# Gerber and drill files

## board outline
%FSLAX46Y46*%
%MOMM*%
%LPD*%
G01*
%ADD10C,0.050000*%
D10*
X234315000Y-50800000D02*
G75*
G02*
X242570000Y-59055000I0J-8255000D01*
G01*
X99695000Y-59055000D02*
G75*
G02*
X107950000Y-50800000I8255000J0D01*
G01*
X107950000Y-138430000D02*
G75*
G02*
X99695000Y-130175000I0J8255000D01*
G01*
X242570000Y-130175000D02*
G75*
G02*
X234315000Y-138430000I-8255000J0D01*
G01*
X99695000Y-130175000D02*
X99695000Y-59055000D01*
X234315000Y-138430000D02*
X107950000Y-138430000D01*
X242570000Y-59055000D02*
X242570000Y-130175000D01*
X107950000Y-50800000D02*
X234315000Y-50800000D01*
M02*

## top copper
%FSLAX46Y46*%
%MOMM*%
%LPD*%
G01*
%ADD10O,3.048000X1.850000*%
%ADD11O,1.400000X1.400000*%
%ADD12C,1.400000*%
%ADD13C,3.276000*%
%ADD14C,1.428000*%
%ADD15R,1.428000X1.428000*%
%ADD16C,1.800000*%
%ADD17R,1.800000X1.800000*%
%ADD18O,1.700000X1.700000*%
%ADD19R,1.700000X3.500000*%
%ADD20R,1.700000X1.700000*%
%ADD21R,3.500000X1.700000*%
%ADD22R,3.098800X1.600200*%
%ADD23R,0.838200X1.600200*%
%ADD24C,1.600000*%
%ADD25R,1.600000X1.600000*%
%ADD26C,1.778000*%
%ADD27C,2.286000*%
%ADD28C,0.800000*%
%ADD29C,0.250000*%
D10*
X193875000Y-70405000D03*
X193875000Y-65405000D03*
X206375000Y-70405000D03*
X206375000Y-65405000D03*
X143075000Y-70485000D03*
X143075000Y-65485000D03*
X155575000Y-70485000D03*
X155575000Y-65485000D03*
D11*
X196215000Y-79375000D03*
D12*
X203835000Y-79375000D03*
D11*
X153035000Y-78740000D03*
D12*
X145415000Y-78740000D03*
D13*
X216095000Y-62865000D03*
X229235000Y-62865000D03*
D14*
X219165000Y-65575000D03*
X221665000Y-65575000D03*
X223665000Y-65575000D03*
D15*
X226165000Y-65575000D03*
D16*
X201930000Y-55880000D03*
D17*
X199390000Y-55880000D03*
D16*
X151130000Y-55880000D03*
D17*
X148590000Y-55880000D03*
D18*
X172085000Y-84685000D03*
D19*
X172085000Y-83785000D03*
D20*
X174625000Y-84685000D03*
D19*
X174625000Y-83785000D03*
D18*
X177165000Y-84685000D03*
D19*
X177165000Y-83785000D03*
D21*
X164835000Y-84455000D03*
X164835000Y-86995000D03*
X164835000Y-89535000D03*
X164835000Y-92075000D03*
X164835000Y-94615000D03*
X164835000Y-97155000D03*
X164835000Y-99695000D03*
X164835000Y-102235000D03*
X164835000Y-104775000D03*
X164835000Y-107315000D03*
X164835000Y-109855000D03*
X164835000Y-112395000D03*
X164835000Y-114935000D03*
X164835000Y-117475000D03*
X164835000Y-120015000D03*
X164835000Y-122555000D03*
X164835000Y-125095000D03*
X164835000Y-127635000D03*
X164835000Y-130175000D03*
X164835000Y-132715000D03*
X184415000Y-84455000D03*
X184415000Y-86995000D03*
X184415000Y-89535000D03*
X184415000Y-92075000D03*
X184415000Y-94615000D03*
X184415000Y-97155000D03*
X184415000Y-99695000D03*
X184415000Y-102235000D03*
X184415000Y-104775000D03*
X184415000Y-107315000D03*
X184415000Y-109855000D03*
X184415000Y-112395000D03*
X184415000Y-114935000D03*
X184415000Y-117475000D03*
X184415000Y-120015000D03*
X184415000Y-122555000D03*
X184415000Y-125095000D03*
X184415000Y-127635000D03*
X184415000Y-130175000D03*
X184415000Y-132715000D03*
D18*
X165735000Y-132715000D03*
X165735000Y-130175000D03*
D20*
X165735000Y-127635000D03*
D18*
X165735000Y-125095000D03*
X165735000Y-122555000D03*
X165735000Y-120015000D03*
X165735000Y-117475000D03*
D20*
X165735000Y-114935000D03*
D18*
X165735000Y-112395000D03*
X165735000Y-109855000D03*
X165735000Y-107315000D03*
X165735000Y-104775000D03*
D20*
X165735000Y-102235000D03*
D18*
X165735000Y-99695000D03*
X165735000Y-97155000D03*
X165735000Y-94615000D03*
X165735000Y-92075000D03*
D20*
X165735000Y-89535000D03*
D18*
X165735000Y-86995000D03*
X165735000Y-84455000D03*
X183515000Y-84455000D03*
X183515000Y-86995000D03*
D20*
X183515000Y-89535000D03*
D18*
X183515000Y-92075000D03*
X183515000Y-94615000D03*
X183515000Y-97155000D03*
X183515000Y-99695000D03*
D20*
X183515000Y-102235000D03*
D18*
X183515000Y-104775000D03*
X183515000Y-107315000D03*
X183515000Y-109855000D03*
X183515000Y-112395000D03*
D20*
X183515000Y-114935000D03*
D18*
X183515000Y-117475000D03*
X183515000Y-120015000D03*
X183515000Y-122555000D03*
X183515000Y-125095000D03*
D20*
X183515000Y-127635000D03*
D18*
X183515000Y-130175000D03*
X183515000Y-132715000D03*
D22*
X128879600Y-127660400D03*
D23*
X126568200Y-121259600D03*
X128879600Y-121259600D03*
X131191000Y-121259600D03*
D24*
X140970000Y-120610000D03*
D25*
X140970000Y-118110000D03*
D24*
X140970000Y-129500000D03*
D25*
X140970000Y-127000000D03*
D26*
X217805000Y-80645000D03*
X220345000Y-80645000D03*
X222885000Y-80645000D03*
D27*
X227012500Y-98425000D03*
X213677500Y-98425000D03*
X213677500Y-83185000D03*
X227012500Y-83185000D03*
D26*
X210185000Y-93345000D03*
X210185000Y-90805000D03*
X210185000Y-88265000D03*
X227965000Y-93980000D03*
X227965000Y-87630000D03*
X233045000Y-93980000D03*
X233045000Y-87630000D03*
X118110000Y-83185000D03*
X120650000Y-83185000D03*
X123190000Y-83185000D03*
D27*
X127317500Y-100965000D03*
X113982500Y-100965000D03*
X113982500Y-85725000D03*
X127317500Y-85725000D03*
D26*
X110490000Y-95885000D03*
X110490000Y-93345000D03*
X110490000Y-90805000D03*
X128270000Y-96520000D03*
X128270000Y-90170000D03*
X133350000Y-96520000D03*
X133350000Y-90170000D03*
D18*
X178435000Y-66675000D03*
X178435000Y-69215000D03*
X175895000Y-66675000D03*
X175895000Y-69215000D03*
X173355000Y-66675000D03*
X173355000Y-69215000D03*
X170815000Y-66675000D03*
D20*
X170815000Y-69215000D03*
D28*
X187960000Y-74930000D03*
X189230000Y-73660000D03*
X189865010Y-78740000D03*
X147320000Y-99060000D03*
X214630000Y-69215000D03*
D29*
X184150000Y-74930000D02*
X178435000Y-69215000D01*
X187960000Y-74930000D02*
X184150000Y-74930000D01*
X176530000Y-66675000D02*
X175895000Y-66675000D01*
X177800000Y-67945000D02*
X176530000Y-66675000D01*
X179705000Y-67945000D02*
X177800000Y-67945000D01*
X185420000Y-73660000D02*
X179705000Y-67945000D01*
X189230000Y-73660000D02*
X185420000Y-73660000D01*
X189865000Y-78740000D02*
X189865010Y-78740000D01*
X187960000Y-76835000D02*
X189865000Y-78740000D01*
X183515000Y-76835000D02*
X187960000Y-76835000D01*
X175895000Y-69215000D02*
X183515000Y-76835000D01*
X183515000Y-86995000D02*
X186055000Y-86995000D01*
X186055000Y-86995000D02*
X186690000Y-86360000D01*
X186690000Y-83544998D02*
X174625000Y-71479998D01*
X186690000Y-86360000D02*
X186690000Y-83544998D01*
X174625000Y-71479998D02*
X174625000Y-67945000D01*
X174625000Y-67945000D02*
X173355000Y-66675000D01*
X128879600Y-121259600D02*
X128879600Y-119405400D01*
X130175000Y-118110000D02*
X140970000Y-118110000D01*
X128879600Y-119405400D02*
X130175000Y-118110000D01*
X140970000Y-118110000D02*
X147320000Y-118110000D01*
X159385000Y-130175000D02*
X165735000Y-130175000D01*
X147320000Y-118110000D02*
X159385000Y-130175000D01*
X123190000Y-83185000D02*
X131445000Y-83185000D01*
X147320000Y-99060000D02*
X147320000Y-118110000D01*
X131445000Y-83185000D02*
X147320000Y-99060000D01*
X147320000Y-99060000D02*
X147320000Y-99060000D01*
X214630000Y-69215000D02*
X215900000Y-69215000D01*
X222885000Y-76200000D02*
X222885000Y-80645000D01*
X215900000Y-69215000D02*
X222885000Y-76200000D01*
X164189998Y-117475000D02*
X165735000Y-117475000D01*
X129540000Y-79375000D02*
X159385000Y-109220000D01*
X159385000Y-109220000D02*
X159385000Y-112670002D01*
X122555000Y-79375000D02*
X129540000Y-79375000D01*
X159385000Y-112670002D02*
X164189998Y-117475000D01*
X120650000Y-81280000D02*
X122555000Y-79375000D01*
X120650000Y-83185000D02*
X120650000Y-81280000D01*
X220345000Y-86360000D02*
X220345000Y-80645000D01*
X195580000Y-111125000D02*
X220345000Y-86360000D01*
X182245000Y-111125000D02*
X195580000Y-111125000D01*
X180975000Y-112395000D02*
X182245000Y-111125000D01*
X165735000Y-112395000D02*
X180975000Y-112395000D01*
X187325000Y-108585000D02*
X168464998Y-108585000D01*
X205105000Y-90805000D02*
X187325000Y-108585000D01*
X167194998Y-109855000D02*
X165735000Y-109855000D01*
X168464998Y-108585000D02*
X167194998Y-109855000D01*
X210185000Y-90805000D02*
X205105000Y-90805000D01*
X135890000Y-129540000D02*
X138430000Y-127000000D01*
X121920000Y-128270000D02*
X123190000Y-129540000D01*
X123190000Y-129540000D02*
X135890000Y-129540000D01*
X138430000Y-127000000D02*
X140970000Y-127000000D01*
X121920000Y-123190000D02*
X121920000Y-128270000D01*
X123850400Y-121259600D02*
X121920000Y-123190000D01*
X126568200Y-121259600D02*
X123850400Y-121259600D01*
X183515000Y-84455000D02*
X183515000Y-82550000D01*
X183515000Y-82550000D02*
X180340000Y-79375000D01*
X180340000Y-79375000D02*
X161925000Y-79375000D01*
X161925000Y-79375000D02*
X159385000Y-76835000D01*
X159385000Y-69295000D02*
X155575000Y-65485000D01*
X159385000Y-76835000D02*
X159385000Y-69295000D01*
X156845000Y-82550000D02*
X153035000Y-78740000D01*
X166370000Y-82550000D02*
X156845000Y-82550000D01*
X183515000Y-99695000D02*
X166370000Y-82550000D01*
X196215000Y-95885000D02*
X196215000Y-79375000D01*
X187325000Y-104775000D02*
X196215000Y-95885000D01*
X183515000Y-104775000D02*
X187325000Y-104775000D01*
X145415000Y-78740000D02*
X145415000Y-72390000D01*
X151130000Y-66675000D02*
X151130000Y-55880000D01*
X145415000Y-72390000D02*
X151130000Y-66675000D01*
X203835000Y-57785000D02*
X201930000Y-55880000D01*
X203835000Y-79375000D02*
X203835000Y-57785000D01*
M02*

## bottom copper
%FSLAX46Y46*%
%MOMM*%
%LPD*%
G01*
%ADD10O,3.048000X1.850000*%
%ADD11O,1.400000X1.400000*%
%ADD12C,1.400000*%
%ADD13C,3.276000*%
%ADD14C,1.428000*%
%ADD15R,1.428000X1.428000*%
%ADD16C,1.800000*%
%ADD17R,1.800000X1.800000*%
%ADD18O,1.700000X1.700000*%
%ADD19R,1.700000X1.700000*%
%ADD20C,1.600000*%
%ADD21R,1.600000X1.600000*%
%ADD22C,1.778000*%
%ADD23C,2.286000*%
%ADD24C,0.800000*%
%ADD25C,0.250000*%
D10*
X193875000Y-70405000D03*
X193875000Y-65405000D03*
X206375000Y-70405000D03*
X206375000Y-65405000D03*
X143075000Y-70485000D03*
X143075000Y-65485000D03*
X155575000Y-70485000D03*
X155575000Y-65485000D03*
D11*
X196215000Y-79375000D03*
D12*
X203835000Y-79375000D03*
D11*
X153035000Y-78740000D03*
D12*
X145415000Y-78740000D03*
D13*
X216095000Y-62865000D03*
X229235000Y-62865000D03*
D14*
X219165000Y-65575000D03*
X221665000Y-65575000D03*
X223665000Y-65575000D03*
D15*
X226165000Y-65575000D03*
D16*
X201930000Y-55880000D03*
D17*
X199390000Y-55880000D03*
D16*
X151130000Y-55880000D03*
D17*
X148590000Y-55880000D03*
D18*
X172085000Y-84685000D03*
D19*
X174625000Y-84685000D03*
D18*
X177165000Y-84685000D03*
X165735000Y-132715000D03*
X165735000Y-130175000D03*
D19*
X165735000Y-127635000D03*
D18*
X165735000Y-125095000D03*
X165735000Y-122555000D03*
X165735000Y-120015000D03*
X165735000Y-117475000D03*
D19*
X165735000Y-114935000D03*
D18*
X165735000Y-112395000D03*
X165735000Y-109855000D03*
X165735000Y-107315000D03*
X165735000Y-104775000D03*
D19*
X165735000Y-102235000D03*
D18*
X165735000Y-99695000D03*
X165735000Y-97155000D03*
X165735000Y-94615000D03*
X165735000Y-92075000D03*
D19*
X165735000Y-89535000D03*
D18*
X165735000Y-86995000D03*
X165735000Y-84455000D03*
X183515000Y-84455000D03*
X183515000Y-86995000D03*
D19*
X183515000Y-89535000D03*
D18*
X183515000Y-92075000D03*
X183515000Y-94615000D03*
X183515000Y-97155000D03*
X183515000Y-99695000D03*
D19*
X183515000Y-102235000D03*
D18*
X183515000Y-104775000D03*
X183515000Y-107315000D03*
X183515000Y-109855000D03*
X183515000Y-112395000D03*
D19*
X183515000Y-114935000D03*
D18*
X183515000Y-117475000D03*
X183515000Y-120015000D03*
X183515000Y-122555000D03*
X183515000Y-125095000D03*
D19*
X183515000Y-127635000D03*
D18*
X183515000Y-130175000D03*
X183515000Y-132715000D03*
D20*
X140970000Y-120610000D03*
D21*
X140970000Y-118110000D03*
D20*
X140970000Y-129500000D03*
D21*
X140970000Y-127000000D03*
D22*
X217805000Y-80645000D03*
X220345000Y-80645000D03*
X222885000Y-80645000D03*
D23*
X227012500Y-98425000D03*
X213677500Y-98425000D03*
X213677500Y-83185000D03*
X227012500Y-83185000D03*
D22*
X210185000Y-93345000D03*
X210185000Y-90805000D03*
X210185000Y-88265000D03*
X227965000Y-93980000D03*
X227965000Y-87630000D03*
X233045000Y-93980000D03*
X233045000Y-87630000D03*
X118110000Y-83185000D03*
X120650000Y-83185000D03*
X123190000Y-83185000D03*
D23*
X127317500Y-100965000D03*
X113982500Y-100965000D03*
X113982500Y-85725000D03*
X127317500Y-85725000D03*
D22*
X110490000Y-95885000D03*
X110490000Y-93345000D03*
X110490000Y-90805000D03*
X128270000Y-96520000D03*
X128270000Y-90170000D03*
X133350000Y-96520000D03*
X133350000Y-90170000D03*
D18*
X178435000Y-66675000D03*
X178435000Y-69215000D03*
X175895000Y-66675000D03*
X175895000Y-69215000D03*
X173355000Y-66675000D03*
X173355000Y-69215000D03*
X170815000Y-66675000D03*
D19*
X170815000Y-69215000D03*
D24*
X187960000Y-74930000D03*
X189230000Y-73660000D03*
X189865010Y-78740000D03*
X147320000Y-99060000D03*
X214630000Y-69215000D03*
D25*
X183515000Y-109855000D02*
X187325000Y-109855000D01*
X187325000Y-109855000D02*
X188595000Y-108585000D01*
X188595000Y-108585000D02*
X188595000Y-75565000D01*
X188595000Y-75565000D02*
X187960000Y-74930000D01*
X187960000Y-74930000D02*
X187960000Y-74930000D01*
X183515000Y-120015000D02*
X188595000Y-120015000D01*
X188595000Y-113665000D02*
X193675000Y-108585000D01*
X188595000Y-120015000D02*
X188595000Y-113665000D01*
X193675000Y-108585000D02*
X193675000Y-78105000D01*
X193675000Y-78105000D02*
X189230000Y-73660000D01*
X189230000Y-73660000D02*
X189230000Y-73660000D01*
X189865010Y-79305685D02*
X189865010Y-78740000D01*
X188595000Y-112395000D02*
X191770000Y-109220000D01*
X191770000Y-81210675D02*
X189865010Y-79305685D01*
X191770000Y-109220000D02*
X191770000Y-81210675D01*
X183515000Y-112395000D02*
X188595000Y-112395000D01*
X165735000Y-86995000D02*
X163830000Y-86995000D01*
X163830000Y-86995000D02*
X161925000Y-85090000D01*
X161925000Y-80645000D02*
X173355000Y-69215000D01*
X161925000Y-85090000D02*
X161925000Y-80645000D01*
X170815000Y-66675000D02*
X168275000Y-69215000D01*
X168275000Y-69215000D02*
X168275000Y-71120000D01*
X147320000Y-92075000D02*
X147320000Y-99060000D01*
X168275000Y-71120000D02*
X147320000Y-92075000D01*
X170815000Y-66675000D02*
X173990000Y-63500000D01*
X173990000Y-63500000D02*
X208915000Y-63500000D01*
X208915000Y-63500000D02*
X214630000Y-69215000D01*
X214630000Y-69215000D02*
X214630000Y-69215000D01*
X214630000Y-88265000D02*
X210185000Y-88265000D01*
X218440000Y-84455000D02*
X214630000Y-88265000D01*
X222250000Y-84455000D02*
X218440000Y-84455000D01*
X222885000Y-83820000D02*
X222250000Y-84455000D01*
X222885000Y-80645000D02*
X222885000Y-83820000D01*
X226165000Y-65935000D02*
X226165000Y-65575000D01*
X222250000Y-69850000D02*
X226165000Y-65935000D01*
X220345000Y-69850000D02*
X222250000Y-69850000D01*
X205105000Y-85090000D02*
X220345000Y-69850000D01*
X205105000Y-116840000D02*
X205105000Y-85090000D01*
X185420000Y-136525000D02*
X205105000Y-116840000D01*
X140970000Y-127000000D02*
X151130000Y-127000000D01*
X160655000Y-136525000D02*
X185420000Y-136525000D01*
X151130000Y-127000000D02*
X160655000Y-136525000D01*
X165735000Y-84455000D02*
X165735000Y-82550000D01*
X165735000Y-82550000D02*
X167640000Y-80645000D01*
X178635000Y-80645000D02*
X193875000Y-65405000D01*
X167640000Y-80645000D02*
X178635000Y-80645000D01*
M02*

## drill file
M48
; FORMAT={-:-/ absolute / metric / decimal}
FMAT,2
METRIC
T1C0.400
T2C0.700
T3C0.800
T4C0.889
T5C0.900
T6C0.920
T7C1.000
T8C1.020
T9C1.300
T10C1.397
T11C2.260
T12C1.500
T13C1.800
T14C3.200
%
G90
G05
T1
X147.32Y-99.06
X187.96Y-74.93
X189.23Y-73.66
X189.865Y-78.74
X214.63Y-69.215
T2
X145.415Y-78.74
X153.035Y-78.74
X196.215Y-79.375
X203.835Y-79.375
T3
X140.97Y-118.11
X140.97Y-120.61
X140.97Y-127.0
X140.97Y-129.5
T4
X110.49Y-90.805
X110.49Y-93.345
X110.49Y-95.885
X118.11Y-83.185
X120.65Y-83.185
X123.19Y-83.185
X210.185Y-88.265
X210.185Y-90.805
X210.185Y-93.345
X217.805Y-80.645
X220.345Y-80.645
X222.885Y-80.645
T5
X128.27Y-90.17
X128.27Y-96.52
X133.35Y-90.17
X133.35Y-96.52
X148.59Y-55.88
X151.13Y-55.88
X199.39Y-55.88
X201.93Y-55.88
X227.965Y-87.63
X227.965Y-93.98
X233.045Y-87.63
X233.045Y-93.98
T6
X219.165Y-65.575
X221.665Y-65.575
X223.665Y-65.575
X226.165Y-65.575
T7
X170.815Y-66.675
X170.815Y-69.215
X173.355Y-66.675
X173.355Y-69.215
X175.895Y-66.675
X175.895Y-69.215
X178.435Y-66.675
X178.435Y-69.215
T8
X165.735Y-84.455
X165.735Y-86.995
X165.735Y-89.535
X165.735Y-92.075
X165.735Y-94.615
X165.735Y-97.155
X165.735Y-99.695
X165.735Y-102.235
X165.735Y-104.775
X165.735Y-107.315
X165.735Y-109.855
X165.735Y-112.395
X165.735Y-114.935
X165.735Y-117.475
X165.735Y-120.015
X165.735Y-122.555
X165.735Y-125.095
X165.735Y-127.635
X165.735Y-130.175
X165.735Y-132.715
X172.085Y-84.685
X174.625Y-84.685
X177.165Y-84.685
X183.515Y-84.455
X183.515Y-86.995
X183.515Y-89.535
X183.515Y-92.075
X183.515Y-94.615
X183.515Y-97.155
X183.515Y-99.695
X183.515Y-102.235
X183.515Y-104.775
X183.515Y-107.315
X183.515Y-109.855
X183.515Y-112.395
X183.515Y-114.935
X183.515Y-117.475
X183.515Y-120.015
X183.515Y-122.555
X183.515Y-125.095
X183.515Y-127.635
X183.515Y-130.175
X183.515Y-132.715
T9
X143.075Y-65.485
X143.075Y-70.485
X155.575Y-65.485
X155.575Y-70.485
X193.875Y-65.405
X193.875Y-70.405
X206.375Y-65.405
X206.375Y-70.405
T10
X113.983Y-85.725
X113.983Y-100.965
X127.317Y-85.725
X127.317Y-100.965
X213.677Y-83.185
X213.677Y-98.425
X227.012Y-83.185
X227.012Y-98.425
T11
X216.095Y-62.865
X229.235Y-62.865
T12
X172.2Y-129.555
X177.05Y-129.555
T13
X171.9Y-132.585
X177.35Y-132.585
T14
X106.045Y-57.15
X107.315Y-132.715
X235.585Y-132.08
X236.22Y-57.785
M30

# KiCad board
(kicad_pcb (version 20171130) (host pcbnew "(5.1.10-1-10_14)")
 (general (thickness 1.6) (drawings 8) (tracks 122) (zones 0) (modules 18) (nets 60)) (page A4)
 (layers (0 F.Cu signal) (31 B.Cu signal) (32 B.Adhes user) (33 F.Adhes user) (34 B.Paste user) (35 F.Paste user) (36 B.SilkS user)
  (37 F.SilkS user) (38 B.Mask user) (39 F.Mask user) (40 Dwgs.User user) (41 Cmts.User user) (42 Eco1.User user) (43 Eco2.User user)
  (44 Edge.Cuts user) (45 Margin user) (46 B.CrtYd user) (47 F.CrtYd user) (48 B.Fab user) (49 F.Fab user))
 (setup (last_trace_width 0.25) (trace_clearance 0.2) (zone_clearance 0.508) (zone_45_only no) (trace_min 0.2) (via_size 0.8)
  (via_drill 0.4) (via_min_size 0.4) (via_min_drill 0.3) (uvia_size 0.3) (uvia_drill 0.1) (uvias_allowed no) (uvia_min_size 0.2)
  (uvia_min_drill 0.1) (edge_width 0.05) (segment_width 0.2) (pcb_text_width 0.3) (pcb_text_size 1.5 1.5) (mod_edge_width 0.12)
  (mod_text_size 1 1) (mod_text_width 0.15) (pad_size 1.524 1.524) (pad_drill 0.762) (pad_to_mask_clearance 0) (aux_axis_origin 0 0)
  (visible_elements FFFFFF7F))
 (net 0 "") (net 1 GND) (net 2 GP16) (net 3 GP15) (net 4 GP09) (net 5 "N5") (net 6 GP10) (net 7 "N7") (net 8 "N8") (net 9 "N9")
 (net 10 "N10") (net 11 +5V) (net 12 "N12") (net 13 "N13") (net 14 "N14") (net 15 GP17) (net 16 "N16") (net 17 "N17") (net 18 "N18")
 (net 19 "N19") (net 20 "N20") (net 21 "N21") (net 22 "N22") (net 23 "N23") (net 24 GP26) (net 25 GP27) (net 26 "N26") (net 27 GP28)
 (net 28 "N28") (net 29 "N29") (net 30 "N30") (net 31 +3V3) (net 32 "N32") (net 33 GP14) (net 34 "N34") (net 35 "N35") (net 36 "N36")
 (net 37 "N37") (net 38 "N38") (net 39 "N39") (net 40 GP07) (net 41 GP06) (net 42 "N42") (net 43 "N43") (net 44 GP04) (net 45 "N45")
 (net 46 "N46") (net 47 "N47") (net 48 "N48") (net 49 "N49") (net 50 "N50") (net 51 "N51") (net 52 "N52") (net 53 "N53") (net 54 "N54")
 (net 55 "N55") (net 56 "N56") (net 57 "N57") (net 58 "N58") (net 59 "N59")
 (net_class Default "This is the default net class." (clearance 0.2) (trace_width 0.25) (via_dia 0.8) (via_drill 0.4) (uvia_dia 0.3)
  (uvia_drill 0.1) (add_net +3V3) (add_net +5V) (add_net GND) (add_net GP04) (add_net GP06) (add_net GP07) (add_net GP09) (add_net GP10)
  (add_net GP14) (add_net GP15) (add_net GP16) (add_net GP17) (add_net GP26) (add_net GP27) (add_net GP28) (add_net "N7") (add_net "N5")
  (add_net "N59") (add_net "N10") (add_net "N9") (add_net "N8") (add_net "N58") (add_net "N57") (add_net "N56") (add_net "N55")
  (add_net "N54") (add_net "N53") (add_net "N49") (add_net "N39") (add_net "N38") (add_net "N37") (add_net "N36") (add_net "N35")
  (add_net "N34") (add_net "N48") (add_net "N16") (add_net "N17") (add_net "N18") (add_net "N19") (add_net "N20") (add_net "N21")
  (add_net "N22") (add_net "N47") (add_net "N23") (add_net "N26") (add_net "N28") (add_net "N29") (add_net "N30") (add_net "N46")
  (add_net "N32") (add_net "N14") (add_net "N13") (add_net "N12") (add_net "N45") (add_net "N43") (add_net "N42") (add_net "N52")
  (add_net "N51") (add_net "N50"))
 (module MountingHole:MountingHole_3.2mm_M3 (layer F.Cu) (at 106.045 57.15)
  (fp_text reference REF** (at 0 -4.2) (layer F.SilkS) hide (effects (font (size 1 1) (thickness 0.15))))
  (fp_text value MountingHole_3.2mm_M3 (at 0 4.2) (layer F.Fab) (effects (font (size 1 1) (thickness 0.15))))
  (pad 1 np_thru_hole circle (at 0 0) (size 3.2 3.2) (drill 3.2) (layers *.Cu *.Mask)))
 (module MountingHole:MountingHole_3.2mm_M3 (layer F.Cu) (at 107.315 132.715)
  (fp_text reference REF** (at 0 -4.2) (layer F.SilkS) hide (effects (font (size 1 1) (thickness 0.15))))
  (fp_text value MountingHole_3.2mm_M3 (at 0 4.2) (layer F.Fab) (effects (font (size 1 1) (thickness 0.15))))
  (pad 1 np_thru_hole circle (at 0 0) (size 3.2 3.2) (drill 3.2) (layers *.Cu *.Mask)))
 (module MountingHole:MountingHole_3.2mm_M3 (layer F.Cu) (at 235.585 132.08)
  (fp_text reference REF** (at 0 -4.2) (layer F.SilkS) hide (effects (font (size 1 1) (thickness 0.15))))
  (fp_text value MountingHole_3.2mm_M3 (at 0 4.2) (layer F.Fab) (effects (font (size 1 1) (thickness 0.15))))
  (pad 1 np_thru_hole circle (at 0 0) (size 3.2 3.2) (drill 3.2) (layers *.Cu *.Mask)))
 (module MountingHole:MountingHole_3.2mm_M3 (layer F.Cu) (at 236.22 57.785)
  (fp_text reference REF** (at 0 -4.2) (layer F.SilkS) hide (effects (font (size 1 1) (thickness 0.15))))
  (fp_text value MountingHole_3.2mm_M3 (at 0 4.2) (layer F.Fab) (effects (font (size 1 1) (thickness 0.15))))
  (pad 1 np_thru_hole circle (at 0 0) (size 3.2 3.2) (drill 3.2) (layers *.Cu *.Mask)))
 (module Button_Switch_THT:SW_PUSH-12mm (layer F.Cu) (at 193.875 65.405)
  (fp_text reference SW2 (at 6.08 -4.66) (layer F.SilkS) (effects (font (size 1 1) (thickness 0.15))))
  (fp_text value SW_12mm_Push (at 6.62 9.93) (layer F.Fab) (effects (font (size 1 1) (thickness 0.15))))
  (pad 2 thru_hole oval (at 0 5) (size 3.048 1.85) (drill 1.3) (layers *.Cu *.Mask) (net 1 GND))
  (pad 1 thru_hole oval (at 0 0) (size 3.048 1.85) (drill 1.3) (layers *.Cu *.Mask) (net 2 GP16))
  (pad 2 thru_hole oval (at 12.5 5) (size 3.048 1.85) (drill 1.3) (layers *.Cu *.Mask) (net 1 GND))
  (pad 1 thru_hole oval (at 12.5 0) (size 3.048 1.85) (drill 1.3) (layers *.Cu *.Mask) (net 2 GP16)))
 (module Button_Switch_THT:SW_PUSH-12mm (layer F.Cu) (at 143.075 65.485)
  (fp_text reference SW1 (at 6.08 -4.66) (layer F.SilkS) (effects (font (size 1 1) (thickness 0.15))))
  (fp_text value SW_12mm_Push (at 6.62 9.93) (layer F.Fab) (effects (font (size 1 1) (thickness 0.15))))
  (pad 2 thru_hole oval (at 0 5) (size 3.048 1.85) (drill 1.3) (layers *.Cu *.Mask) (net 1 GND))
  (pad 1 thru_hole oval (at 0 0) (size 3.048 1.85) (drill 1.3) (layers *.Cu *.Mask) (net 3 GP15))
  (pad 2 thru_hole oval (at 12.5 5) (size 3.048 1.85) (drill 1.3) (layers *.Cu *.Mask) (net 1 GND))
  (pad 1 thru_hole oval (at 12.5 0) (size 3.048 1.85) (drill 1.3) (layers *.Cu *.Mask) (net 3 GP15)))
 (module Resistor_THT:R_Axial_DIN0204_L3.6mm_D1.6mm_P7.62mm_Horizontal (layer F.Cu) (at 203.835 79.375 180)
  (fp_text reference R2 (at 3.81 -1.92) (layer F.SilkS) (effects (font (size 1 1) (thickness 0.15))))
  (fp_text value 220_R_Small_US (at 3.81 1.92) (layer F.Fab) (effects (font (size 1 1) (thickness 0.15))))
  (pad 2 thru_hole oval (at 7.62 0 180) (size 1.4 1.4) (drill 0.7) (layers *.Cu *.Mask) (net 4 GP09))
  (pad 1 thru_hole circle (at 0 0 180) (size 1.4 1.4) (drill 0.7) (layers *.Cu *.Mask) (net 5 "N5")))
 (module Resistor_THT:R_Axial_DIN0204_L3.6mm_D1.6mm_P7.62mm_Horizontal (layer F.Cu) (at 145.415 78.74)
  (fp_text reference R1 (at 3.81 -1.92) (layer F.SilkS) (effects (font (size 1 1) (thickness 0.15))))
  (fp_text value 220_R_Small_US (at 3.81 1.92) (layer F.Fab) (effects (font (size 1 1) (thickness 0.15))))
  (pad 2 thru_hole oval (at 7.62 0) (size 1.4 1.4) (drill 0.7) (layers *.Cu *.Mask) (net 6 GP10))
  (pad 1 thru_hole circle (at 0 0) (size 1.4 1.4) (drill 0.7) (layers *.Cu *.Mask) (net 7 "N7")))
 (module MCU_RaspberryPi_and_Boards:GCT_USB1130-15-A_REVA (layer F.Cu) (at 222.665 62.865 180)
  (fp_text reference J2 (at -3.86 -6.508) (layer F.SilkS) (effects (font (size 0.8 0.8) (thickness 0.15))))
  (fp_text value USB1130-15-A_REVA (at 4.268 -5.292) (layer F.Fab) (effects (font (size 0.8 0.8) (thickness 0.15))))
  (pad S2 thru_hole circle (at 6.57 0 180) (size 3.276 3.276) (drill 2.26) (layers *.Cu *.Mask) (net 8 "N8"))
  (pad S1 thru_hole circle (at -6.57 0 180) (size 3.276 3.276) (drill 2.26) (layers *.Cu *.Mask) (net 8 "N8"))
  (pad 4 thru_hole circle (at 3.5 -2.71 180) (size 1.428 1.428) (drill 0.92) (layers *.Cu *.Mask) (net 1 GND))
  (pad 3 thru_hole circle (at 1 -2.71 180) (size 1.428 1.428) (drill 0.92) (layers *.Cu *.Mask) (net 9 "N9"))
  (pad 2 thru_hole circle (at -1 -2.71 180) (size 1.428 1.428) (drill 0.92) (layers *.Cu *.Mask) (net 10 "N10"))
  (pad 1 thru_hole rect (at -3.5 -2.71 180) (size 1.428 1.428) (drill 0.92) (layers *.Cu *.Mask) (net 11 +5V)))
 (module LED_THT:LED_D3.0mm (layer F.Cu) (at 199.39 55.88)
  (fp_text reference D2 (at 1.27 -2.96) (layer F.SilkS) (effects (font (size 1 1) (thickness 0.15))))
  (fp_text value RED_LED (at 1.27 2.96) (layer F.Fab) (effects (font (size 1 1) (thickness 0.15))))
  (pad 2 thru_hole circle (at 2.54 0) (size 1.8 1.8) (drill 0.9) (layers *.Cu *.Mask) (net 5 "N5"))
  (pad 1 thru_hole rect (at 0 0) (size 1.8 1.8) (drill 0.9) (layers *.Cu *.Mask) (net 1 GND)))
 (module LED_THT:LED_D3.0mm (layer F.Cu) (at 148.59 55.88)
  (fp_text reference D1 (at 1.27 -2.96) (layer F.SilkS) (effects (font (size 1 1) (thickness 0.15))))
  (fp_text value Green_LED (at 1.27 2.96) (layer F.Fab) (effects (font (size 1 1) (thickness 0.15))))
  (pad 2 thru_hole circle (at 2.54 0) (size 1.8 1.8) (drill 0.9) (layers *.Cu *.Mask) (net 7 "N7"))
  (pad 1 thru_hole rect (at 0 0) (size 1.8 1.8) (drill 0.9) (layers *.Cu *.Mask) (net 1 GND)))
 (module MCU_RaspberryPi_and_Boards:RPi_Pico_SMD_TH (layer F.Cu) (at 174.625 108.585 180)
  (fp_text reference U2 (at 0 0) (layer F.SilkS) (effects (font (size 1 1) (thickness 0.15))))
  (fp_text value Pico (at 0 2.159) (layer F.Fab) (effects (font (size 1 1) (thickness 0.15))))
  (pad 43 thru_hole oval (at 2.54 23.9 180) (size 1.7 1.7) (drill 1.02) (layers *.Cu *.Mask) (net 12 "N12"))
  (pad 43 smd rect (at 2.54 23.9 270) (size 3.5 1.7) (drill (offset -0.9 0)) (layers F.Cu F.Mask) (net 12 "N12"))
  (pad 42 thru_hole rect (at 0 23.9 180) (size 1.7 1.7) (drill 1.02) (layers *.Cu *.Mask) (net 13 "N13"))
  (pad 42 smd rect (at 0 23.9 270) (size 3.5 1.7) (drill (offset -0.9 0)) (layers F.Cu F.Mask) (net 13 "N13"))
  (pad 41 thru_hole oval (at -2.54 23.9 180) (size 1.7 1.7) (drill 1.02) (layers *.Cu *.Mask) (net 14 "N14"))
  (pad 41 smd rect (at -2.54 23.9 270) (size 3.5 1.7) (drill (offset -0.9 0)) (layers F.Cu F.Mask) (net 14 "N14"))
  (pad "" np_thru_hole oval (at 2.425 -20.97 180) (size 1.5 1.5) (drill 1.5) (layers *.Cu *.Mask))
  (pad "" np_thru_hole oval (at -2.425 -20.97 180) (size 1.5 1.5) (drill 1.5) (layers *.Cu *.Mask))
  (pad "" np_thru_hole oval (at 2.725 -24 180) (size 1.8 1.8) (drill 1.8) (layers *.Cu *.Mask))
  (pad "" np_thru_hole oval (at -2.725 -24 180) (size 1.8 1.8) (drill 1.8) (layers *.Cu *.Mask))
  (pad 21 smd rect (at 8.89 24.13 180) (size 3.5 1.7) (drill (offset 0.9 0)) (layers F.Cu F.Mask) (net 2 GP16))
  (pad 22 smd rect (at 8.89 21.59 180) (size 3.5 1.7) (drill (offset 0.9 0)) (layers F.Cu F.Mask) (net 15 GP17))
  (pad 23 smd rect (at 8.89 19.05 180) (size 3.5 1.7) (drill (offset 0.9 0)) (layers F.Cu F.Mask) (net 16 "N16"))
  (pad 24 smd rect (at 8.89 16.51 180) (size 3.5 1.7) (drill (offset 0.9 0)) (layers F.Cu F.Mask) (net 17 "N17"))
  (pad 25 smd rect (at 8.89 13.97 180) (size 3.5 1.7) (drill (offset 0.9 0)) (layers F.Cu F.Mask) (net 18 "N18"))
  (pad 26 smd rect (at 8.89 11.43 180) (size 3.5 1.7) (drill (offset 0.9 0)) (layers F.Cu F.Mask) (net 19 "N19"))
  (pad 27 smd rect (at 8.89 8.89 180) (size 3.5 1.7) (drill (offset 0.9 0)) (layers F.Cu F.Mask) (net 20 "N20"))
  (pad 28 smd rect (at 8.89 6.35 180) (size 3.5 1.7) (drill (offset 0.9 0)) (layers F.Cu F.Mask) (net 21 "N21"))
  (pad 29 smd rect (at 8.89 3.81 180) (size 3.5 1.7) (drill (offset 0.9 0)) (layers F.Cu F.Mask) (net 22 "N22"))
  (pad 30 smd rect (at 8.89 1.27 180) (size 3.5 1.7) (drill (offset 0.9 0)) (layers F.Cu F.Mask) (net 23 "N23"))
  (pad 31 smd rect (at 8.89 -1.27 180) (size 3.5 1.7) (drill (offset 0.9 0)) (layers F.Cu F.Mask) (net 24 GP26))
  (pad 32 smd rect (at 8.89 -3.81 180) (size 3.5 1.7) (drill (offset 0.9 0)) (layers F.Cu F.Mask) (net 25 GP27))
  (pad 33 smd rect (at 8.89 -6.35 180) (size 3.5 1.7) (drill (offset 0.9 0)) (layers F.Cu F.Mask) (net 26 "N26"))
  (pad 34 smd rect (at 8.89 -8.89 180) (size 3.5 1.7) (drill (offset 0.9 0)) (layers F.Cu F.Mask) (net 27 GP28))
  (pad 35 smd rect (at 8.89 -11.43 180) (size 3.5 1.7) (drill (offset 0.9 0)) (layers F.Cu F.Mask) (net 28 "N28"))
  (pad 36 smd rect (at 8.89 -13.97 180) (size 3.5 1.7) (drill (offset 0.9 0)) (layers F.Cu F.Mask) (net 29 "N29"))
  (pad 37 smd rect (at 8.89 -16.51 180) (size 3.5 1.7) (drill (offset 0.9 0)) (layers F.Cu F.Mask) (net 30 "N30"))
  (pad 38 smd rect (at 8.89 -19.05 180) (size 3.5 1.7) (drill (offset 0.9 0)) (layers F.Cu F.Mask) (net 1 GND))
  (pad 39 smd rect (at 8.89 -21.59 180) (size 3.5 1.7) (drill (offset 0.9 0)) (layers F.Cu F.Mask) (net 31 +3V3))
  (pad 40 smd rect (at 8.89 -24.13 180) (size 3.5 1.7) (drill (offset 0.9 0)) (layers F.Cu F.Mask) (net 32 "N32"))
  (pad 20 smd rect (at -8.89 24.13 180) (size 3.5 1.7) (drill (offset -0.9 0)) (layers F.Cu F.Mask) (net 3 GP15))
  (pad 19 smd rect (at -8.89 21.59 180) (size 3.5 1.7) (drill (offset -0.9 0)) (layers F.Cu F.Mask) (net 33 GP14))
  (pad 18 smd rect (at -8.89 19.05 180) (size 3.5 1.7) (drill (offset -0.9 0)) (layers F.Cu F.Mask) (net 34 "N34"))
  (pad 17 smd rect (at -8.89 16.51 180) (size 3.5 1.7) (drill (offset -0.9 0)) (layers F.Cu F.Mask) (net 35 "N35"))
  (pad 16 smd rect (at -8.89 13.97 180) (size 3.5 1.7) (drill (offset -0.9 0)) (layers F.Cu F.Mask) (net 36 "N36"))
  (pad 15 smd rect (at -8.89 11.43 180) (size 3.5 1.7) (drill (offset -0.9 0)) (layers F.Cu F.Mask) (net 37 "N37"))
  (pad 14 smd rect (at -8.89 8.89 180) (size 3.5 1.7) (drill (offset -0.9 0)) (layers F.Cu F.Mask) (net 6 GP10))
  (pad 13 smd rect (at -8.89 6.35 180) (size 3.5 1.7) (drill (offset -0.9 0)) (layers F.Cu F.Mask) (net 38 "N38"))
  (pad 12 smd rect (at -8.89 3.81 180) (size 3.5 1.7) (drill (offset -0.9 0)) (layers F.Cu F.Mask) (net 4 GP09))
  (pad 11 smd rect (at -8.89 1.27 180) (size 3.5 1.7) (drill (offset -0.9 0)) (layers F.Cu F.Mask) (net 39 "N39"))
  (pad 10 smd rect (at -8.89 -1.27 180) (size 3.5 1.7) (drill (offset -0.9 0)) (layers F.Cu F.Mask) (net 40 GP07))
  (pad 9 smd rect (at -8.89 -3.81 180) (size 3.5 1.7) (drill (offset -0.9 0)) (layers F.Cu F.Mask) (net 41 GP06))
  (pad 8 smd rect (at -8.89 -6.35 180) (size 3.5 1.7) (drill (offset -0.9 0)) (layers F.Cu F.Mask) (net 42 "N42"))
  (pad 7 smd rect (at -8.89 -8.89 180) (size 3.5 1.7) (drill (offset -0.9 0)) (layers F.Cu F.Mask) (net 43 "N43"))
  (pad 6 smd rect (at -8.89 -11.43 180) (size 3.5 1.7) (drill (offset -0.9 0)) (layers F.Cu F.Mask) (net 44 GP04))
  (pad 5 smd rect (at -8.89 -13.97 180) (size 3.5 1.7) (drill (offset -0.9 0)) (layers F.Cu F.Mask) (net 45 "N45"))
  (pad 4 smd rect (at -8.89 -16.51 180) (size 3.5 1.7) (drill (offset -0.9 0)) (layers F.Cu F.Mask) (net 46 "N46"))
  (pad 3 smd rect (at -8.89 -19.05 180) (size 3.5 1.7) (drill (offset -0.9 0)) (layers F.Cu F.Mask) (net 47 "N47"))
  (pad 2 smd rect (at -8.89 -21.59 180) (size 3.5 1.7) (drill (offset -0.9 0)) (layers F.Cu F.Mask) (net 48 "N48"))
  (pad 1 smd rect (at -8.89 -24.13 180) (size 3.5 1.7) (drill (offset -0.9 0)) (layers F.Cu F.Mask) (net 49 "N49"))
  (pad 40 thru_hole oval (at 8.89 -24.13 180) (size 1.7 1.7) (drill 1.02) (layers *.Cu *.Mask) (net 32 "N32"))
  (pad 39 thru_hole oval (at 8.89 -21.59 180) (size 1.7 1.7) (drill 1.02) (layers *.Cu *.Mask) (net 31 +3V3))
  (pad 38 thru_hole rect (at 8.89 -19.05 180) (size 1.7 1.7) (drill 1.02) (layers *.Cu *.Mask) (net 1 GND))
  (pad 37 thru_hole oval (at 8.89 -16.51 180) (size 1.7 1.7) (drill 1.02) (layers *.Cu *.Mask) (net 30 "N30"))
  (pad 36 thru_hole oval (at 8.89 -13.97 180) (size 1.7 1.7) (drill 1.02) (layers *.Cu *.Mask) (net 29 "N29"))
  (pad 35 thru_hole oval (at 8.89 -11.43 180) (size 1.7 1.7) (drill 1.02) (layers *.Cu *.Mask) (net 28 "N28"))
  (pad 34 thru_hole oval (at 8.89 -8.89 180) (size 1.7 1.7) (drill 1.02) (layers *.Cu *.Mask) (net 27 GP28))
  (pad 33 thru_hole rect (at 8.89 -6.35 180) (size 1.7 1.7) (drill 1.02) (layers *.Cu *.Mask) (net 26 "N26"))
  (pad 32 thru_hole oval (at 8.89 -3.81 180) (size 1.7 1.7) (drill 1.02) (layers *.Cu *.Mask) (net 25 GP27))
  (pad 31 thru_hole oval (at 8.89 -1.27 180) (size 1.7 1.7) (drill 1.02) (layers *.Cu *.Mask) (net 24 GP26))
  (pad 30 thru_hole oval (at 8.89 1.27 180) (size 1.7 1.7) (drill 1.02) (layers *.Cu *.Mask) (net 23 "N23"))
  (pad 29 thru_hole oval (at 8.89 3.81 180) (size 1.7 1.7) (drill 1.02) (layers *.Cu *.Mask) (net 22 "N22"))
  (pad 28 thru_hole rect (at 8.89 6.35 180) (size 1.7 1.7) (drill 1.02) (layers *.Cu *.Mask) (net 21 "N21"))
  (pad 27 thru_hole oval (at 8.89 8.89 180) (size 1.7 1.7) (drill 1.02) (layers *.Cu *.Mask) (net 20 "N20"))
  (pad 26 thru_hole oval (at 8.89 11.43 180) (size 1.7 1.7) (drill 1.02) (layers *.Cu *.Mask) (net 19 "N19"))
  (pad 25 thru_hole oval (at 8.89 13.97 180) (size 1.7 1.7) (drill 1.02) (layers *.Cu *.Mask) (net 18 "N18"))
  (pad 24 thru_hole oval (at 8.89 16.51 180) (size 1.7 1.7) (drill 1.02) (layers *.Cu *.Mask) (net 17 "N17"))
  (pad 23 thru_hole rect (at 8.89 19.05 180) (size 1.7 1.7) (drill 1.02) (layers *.Cu *.Mask) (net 16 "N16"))
  (pad 22 thru_hole oval (at 8.89 21.59 180) (size 1.7 1.7) (drill 1.02) (layers *.Cu *.Mask) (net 15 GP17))
  (pad 21 thru_hole oval (at 8.89 24.13 180) (size 1.7 1.7) (drill 1.02) (layers *.Cu *.Mask) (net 2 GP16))
  (pad 20 thru_hole oval (at -8.89 24.13 180) (size 1.7 1.7) (drill 1.02) (layers *.Cu *.Mask) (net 3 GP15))
  (pad 19 thru_hole oval (at -8.89 21.59 180) (size 1.7 1.7) (drill 1.02) (layers *.Cu *.Mask) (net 33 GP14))
  (pad 18 thru_hole rect (at -8.89 19.05 180) (size 1.7 1.7) (drill 1.02) (layers *.Cu *.Mask) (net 34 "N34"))
  (pad 17 thru_hole oval (at -8.89 16.51 180) (size 1.7 1.7) (drill 1.02) (layers *.Cu *.Mask) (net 35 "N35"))
  (pad 16 thru_hole oval (at -8.89 13.97 180) (size 1.7 1.7) (drill 1.02) (layers *.Cu *.Mask) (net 36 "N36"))
  (pad 15 thru_hole oval (at -8.89 11.43 180) (size 1.7 1.7) (drill 1.02) (layers *.Cu *.Mask) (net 37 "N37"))
  (pad 14 thru_hole oval (at -8.89 8.89 180) (size 1.7 1.7) (drill 1.02) (layers *.Cu *.Mask) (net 6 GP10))
  (pad 13 thru_hole rect (at -8.89 6.35 180) (size 1.7 1.7) (drill 1.02) (layers *.Cu *.Mask) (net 38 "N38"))
  (pad 12 thru_hole oval (at -8.89 3.81 180) (size 1.7 1.7) (drill 1.02) (layers *.Cu *.Mask) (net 4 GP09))
  (pad 11 thru_hole oval (at -8.89 1.27 180) (size 1.7 1.7) (drill 1.02) (layers *.Cu *.Mask) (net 39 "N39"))
  (pad 10 thru_hole oval (at -8.89 -1.27 180) (size 1.7 1.7) (drill 1.02) (layers *.Cu *.Mask) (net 40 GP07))
  (pad 9 thru_hole oval (at -8.89 -3.81 180) (size 1.7 1.7) (drill 1.02) (layers *.Cu *.Mask) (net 41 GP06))
  (pad 8 thru_hole rect (at -8.89 -6.35 180) (size 1.7 1.7) (drill 1.02) (layers *.Cu *.Mask) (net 42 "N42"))
  (pad 7 thru_hole oval (at -8.89 -8.89 180) (size 1.7 1.7) (drill 1.02) (layers *.Cu *.Mask) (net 43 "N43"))
  (pad 6 thru_hole oval (at -8.89 -11.43 180) (size 1.7 1.7) (drill 1.02) (layers *.Cu *.Mask) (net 44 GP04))
  (pad 5 thru_hole oval (at -8.89 -13.97 180) (size 1.7 1.7) (drill 1.02) (layers *.Cu *.Mask) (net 45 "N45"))
  (pad 4 thru_hole oval (at -8.89 -16.51 180) (size 1.7 1.7) (drill 1.02) (layers *.Cu *.Mask) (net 46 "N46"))
  (pad 3 thru_hole rect (at -8.89 -19.05 180) (size 1.7 1.7) (drill 1.02) (layers *.Cu *.Mask) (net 47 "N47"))
  (pad 2 thru_hole oval (at -8.89 -21.59 180) (size 1.7 1.7) (drill 1.02) (layers *.Cu *.Mask) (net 48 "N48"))
  (pad 1 thru_hole oval (at -8.89 -24.13 180) (size 1.7 1.7) (drill 1.02) (layers *.Cu *.Mask) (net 49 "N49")))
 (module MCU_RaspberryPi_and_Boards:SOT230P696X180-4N (layer F.Cu) (at 128.8796 124.46 270)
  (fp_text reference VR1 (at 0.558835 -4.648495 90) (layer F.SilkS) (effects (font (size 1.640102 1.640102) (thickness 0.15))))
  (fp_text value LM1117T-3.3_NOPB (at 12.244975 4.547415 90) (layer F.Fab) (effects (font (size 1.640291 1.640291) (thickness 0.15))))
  (pad 4 smd rect (at 3.2004 0 270) (size 1.6002 3.0988) (layers F.Cu F.Paste F.Mask))
  (pad 3 smd rect (at -3.2004 2.3114 270) (size 1.6002 0.8382) (layers F.Cu F.Paste F.Mask) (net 11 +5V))
  (pad 2 smd rect (at -3.2004 0 270) (size 1.6002 0.8382) (layers F.Cu F.Paste F.Mask) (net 31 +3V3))
  (pad 1 smd rect (at -3.2004 -2.3114 270) (size 1.6002 0.8382) (layers F.Cu F.Paste F.Mask) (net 1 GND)))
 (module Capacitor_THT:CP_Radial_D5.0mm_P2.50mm (layer F.Cu) (at 140.97 118.11 270)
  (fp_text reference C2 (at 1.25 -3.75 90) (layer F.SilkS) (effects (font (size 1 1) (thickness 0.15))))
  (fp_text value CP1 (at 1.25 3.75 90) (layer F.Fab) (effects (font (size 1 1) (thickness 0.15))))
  (pad 2 thru_hole circle (at 2.5 0 270) (size 1.6 1.6) (drill 0.8) (layers *.Cu *.Mask) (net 1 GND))
  (pad 1 thru_hole rect (at 0 0 270) (size 1.6 1.6) (drill 0.8) (layers *.Cu *.Mask) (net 31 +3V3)))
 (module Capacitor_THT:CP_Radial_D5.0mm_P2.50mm (layer F.Cu) (at 140.97 127 270)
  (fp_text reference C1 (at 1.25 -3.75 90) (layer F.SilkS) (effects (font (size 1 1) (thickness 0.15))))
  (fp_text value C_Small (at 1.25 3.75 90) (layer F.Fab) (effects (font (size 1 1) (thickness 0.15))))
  (pad 2 thru_hole circle (at 2.5 0 270) (size 1.6 1.6) (drill 0.8) (layers *.Cu *.Mask) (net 1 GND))
  (pad 1 thru_hole rect (at 0 0 270) (size 1.6 1.6) (drill 0.8) (layers *.Cu *.Mask) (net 11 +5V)))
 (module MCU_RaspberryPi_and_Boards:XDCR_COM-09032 (layer F.Cu) (at 220.345 90.805 270)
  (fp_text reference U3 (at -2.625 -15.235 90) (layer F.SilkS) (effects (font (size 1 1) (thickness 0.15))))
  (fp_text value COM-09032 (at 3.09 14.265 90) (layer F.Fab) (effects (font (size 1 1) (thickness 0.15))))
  (pad V3 thru_hole circle (at -10.16 2.54 270) (size 1.778 1.778) (drill 0.889) (layers *.Cu *.Mask) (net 1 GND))
  (pad V2 thru_hole circle (at -10.16 0 270) (size 1.778 1.778) (drill 0.889) (layers *.Cu *.Mask) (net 25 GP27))
  (pad V1 thru_hole circle (at -10.16 -2.54 270) (size 1.778 1.778) (drill 0.889) (layers *.Cu *.Mask) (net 31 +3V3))
  (pad S4 thru_hole circle (at 7.62 -6.6675 270) (size 2.286 2.286) (drill 1.397) (layers *.Cu *.Mask) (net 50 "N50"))
  (pad S3 thru_hole circle (at 7.62 6.6675 270) (size 2.286 2.286) (drill 1.397) (layers *.Cu *.Mask) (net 50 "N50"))
  (pad S2 thru_hole circle (at -7.62 6.6675 270) (size 2.286 2.286) (drill 1.397) (layers *.Cu *.Mask) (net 50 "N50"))
  (pad S1 thru_hole circle (at -7.62 -6.6675 270) (size 2.286 2.286) (drill 1.397) (layers *.Cu *.Mask) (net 50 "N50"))
  (pad H3 thru_hole circle (at 2.54 10.16 270) (size 1.778 1.778) (drill 0.889) (layers *.Cu *.Mask) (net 1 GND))
  (pad H2 thru_hole circle (at 0 10.16 270) (size 1.778 1.778) (drill 0.889) (layers *.Cu *.Mask) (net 24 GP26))
  (pad H1 thru_hole circle (at -2.54 10.16 270) (size 1.778 1.778) (drill 0.889) (layers *.Cu *.Mask) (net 31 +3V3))
  (pad B2B thru_hole circle (at 3.175 -7.62 270) (size 1.778 1.778) (drill 0.9) (layers *.Cu *.Mask))
  (pad B2A thru_hole circle (at -3.175 -7.62 270) (size 1.778 1.778) (drill 0.9) (layers *.Cu *.Mask) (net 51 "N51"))
  (pad B1B thru_hole circle (at 3.175 -12.7 270) (size 1.778 1.778) (drill 0.9) (layers *.Cu *.Mask))
  (pad B1A thru_hole circle (at -3.175 -12.7 270) (size 1.778 1.778) (drill 0.9) (layers *.Cu *.Mask) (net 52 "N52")))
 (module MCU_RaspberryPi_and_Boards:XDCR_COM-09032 (layer F.Cu) (at 120.65 93.345 270)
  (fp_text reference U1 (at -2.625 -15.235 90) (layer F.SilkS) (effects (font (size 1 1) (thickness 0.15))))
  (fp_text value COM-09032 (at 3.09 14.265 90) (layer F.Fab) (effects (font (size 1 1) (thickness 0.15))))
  (pad V3 thru_hole circle (at -10.16 2.54 270) (size 1.778 1.778) (drill 0.889) (layers *.Cu *.Mask) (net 1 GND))
  (pad V2 thru_hole circle (at -10.16 0 270) (size 1.778 1.778) (drill 0.889) (layers *.Cu *.Mask) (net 27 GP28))
  (pad V1 thru_hole circle (at -10.16 -2.54 270) (size 1.778 1.778) (drill 0.889) (layers *.Cu *.Mask) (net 31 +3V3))
  (pad S4 thru_hole circle (at 7.62 -6.6675 270) (size 2.286 2.286) (drill 1.397) (layers *.Cu *.Mask) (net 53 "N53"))
  (pad S3 thru_hole circle (at 7.62 6.6675 270) (size 2.286 2.286) (drill 1.397) (layers *.Cu *.Mask) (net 53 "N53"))
  (pad S2 thru_hole circle (at -7.62 6.6675 270) (size 2.286 2.286) (drill 1.397) (layers *.Cu *.Mask) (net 53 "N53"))
  (pad S1 thru_hole circle (at -7.62 -6.6675 270) (size 2.286 2.286) (drill 1.397) (layers *.Cu *.Mask) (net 53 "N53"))
  (pad H3 thru_hole circle (at 2.54 10.16 270) (size 1.778 1.778) (drill 0.889) (layers *.Cu *.Mask) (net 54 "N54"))
  (pad H2 thru_hole circle (at 0 10.16 270) (size 1.778 1.778) (drill 0.889) (layers *.Cu *.Mask) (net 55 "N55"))
  (pad H1 thru_hole circle (at -2.54 10.16 270) (size 1.778 1.778) (drill 0.889) (layers *.Cu *.Mask) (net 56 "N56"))
  (pad B2B thru_hole circle (at 3.175 -7.62 270) (size 1.778 1.778) (drill 0.9) (layers *.Cu *.Mask))
  (pad B2A thru_hole circle (at -3.175 -7.62 270) (size 1.778 1.778) (drill 0.9) (layers *.Cu *.Mask) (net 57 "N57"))
  (pad B1B thru_hole circle (at 3.175 -12.7 270) (size 1.778 1.778) (drill 0.9) (layers *.Cu *.Mask))
  (pad B1A thru_hole circle (at -3.175 -12.7 270) (size 1.778 1.778) (drill 0.9) (layers *.Cu *.Mask) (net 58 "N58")))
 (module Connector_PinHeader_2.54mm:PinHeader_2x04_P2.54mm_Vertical (layer F.Cu) (at 170.815 69.215 90)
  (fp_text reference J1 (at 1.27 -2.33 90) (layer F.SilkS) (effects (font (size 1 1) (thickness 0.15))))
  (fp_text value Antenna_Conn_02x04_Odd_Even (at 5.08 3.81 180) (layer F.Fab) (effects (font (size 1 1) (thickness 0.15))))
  (pad 8 thru_hole oval (at 2.54 7.62 90) (size 1.7 1.7) (drill 1) (layers *.Cu *.Mask) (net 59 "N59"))
  (pad 7 thru_hole oval (at 0 7.62 90) (size 1.7 1.7) (drill 1) (layers *.Cu *.Mask) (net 40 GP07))
  (pad 6 thru_hole oval (at 2.54 5.08 90) (size 1.7 1.7) (drill 1) (layers *.Cu *.Mask) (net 44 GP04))
  (pad 5 thru_hole oval (at 0 5.08 90) (size 1.7 1.7) (drill 1) (layers *.Cu *.Mask) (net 41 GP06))
  (pad 4 thru_hole oval (at 2.54 2.54 90) (size 1.7 1.7) (drill 1) (layers *.Cu *.Mask) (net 33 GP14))
  (pad 3 thru_hole oval (at 0 2.54 90) (size 1.7 1.7) (drill 1) (layers *.Cu *.Mask) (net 15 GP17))
  (pad 2 thru_hole oval (at 2.54 0 90) (size 1.7 1.7) (drill 1) (layers *.Cu *.Mask) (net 31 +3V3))
  (pad 1 thru_hole rect (at 0 0 90) (size 1.7 1.7) (drill 1) (layers *.Cu *.Mask) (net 1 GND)))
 (gr_arc (start 234.315 59.055) (end 242.57 59.055) (angle -90) (layer Edge.Cuts) (width 0.05))
 (gr_arc (start 107.95 59.055) (end 107.95 50.8) (angle -90) (layer Edge.Cuts) (width 0.05))
 (gr_arc (start 107.95 130.175) (end 99.695 130.175) (angle -90) (layer Edge.Cuts) (width 0.05))
 (gr_arc (start 234.315 130.175) (end 234.315 138.43) (angle -90) (layer Edge.Cuts) (width 0.05))
 (gr_line (start 99.695 130.175) (end 99.695 59.055) (layer Edge.Cuts) (width 0.05))
 (gr_line (start 234.315 138.43) (end 107.95 138.43) (layer Edge.Cuts) (width 0.05))
 (gr_line (start 242.57 59.055) (end 242.57 130.175) (layer Edge.Cuts) (width 0.05))
 (gr_line (start 107.95 50.8) (end 234.315 50.8) (layer Edge.Cuts) (width 0.05))
 (segment (start 183.515 109.855) (end 187.325 109.855) (width 0.25) (layer B.Cu) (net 40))
 (segment (start 187.325 109.855) (end 188.595 108.585) (width 0.25) (layer B.Cu) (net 40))
 (segment (start 188.595 108.585) (end 188.595 75.565) (width 0.25) (layer B.Cu) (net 40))
 (segment (start 188.595 75.565) (end 187.96 74.93) (width 0.25) (layer B.Cu) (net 40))
 (segment (start 187.96 74.93) (end 187.96 74.93) (width 0.25) (layer B.Cu) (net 40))
 (via (at 187.96 74.93) (size 0.8) (drill 0.4) (layers F.Cu B.Cu) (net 40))
 (segment (start 184.15 74.93) (end 178.435 69.215) (width 0.25) (layer F.Cu) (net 40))
 (segment (start 187.96 74.93) (end 184.15 74.93) (width 0.25) (layer F.Cu) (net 40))
 (segment (start 183.515 120.015) (end 188.595 120.015) (width 0.25) (layer B.Cu) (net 44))
 (segment (start 188.595 113.665) (end 193.675 108.585) (width 0.25) (layer B.Cu) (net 44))
 (segment (start 188.595 120.015) (end 188.595 113.665) (width 0.25) (layer B.Cu) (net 44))
 (segment (start 193.675 108.585) (end 193.675 78.105) (width 0.25) (layer B.Cu) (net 44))
 (segment (start 193.675 78.105) (end 189.23 73.66) (width 0.25) (layer B.Cu) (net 44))
 (segment (start 189.23 73.66) (end 189.23 73.66) (width 0.25) (layer B.Cu) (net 44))
 (via (at 189.23 73.66) (size 0.8) (drill 0.4) (layers F.Cu B.Cu) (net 44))
 (segment (start 176.53 66.675) (end 175.895 66.675) (width 0.25) (layer F.Cu) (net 44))
 (segment (start 177.8 67.945) (end 176.53 66.675) (width 0.25) (layer F.Cu) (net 44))
 (segment (start 179.705 67.945) (end 177.8 67.945) (width 0.25) (layer F.Cu) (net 44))
 (segment (start 185.42 73.66) (end 179.705 67.945) (width 0.25) (layer F.Cu) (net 44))
 (segment (start 189.23 73.66) (end 185.42 73.66) (width 0.25) (layer F.Cu) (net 44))
 (via (at 189.86501 78.74) (size 0.8) (drill 0.4) (layers F.Cu B.Cu) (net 41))
 (segment (start 189.865 78.74) (end 189.86501 78.74) (width 0.25) (layer F.Cu) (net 41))
 (segment (start 187.96 76.835) (end 189.865 78.74) (width 0.25) (layer F.Cu) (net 41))
 (segment (start 183.515 76.835) (end 187.96 76.835) (width 0.25) (layer F.Cu) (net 41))
 (segment (start 175.895 69.215) (end 183.515 76.835) (width 0.25) (layer F.Cu) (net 41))
 (segment (start 189.86501 79.305685) (end 189.86501 78.74) (width 0.25) (layer B.Cu) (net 41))
 (segment (start 188.595 112.395) (end 191.77 109.22) (width 0.25) (layer B.Cu) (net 41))
 (segment (start 191.77 81.210675) (end 189.86501 79.305685) (width 0.25) (layer B.Cu) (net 41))
 (segment (start 191.77 109.22) (end 191.77 81.210675) (width 0.25) (layer B.Cu) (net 41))
 (segment (start 183.515 112.395) (end 188.595 112.395) (width 0.25) (layer B.Cu) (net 41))
 (segment (start 183.515 86.995) (end 186.055 86.995) (width 0.25) (layer F.Cu) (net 33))
 (segment (start 186.055 86.995) (end 186.69 86.36) (width 0.25) (layer F.Cu) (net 33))
 (segment (start 186.69 83.544998) (end 174.625 71.479998) (width 0.25) (layer F.Cu) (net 33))
 (segment (start 186.69 86.36) (end 186.69 83.544998) (width 0.25) (layer F.Cu) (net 33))
 (segment (start 174.625 71.479998) (end 174.625 67.945) (width 0.25) (layer F.Cu) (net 33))
 (segment (start 174.625 67.945) (end 173.355 66.675) (width 0.25) (layer F.Cu) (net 33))
 (segment (start 165.735 86.995) (end 163.83 86.995) (width 0.25) (layer B.Cu) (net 15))
 (segment (start 163.83 86.995) (end 161.925 85.09) (width 0.25) (layer B.Cu) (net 15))
 (segment (start 161.925 80.645) (end 173.355 69.215) (width 0.25) (layer B.Cu) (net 15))
 (segment (start 161.925 85.09) (end 161.925 80.645) (width 0.25) (layer B.Cu) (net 15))
 (segment (start 128.8796 121.2596) (end 128.8796 119.4054) (width 0.25) (layer F.Cu) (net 31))
 (segment (start 130.175 118.11) (end 140.97 118.11) (width 0.25) (layer F.Cu) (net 31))
 (segment (start 128.8796 119.4054) (end 130.175 118.11) (width 0.25) (layer F.Cu) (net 31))
 (segment (start 140.97 118.11) (end 147.32 118.11) (width 0.25) (layer F.Cu) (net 31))
 (segment (start 159.385 130.175) (end 165.735 130.175) (width 0.25) (layer F.Cu) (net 31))
 (segment (start 147.32 118.11) (end 159.385 130.175) (width 0.25) (layer F.Cu) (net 31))
 (segment (start 123.19 83.185) (end 131.445 83.185) (width 0.25) (layer F.Cu) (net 31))
 (segment (start 147.32 99.06) (end 147.32 118.11) (width 0.25) (layer F.Cu) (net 31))
 (segment (start 131.445 83.185) (end 147.32 99.06) (width 0.25) (layer F.Cu) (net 31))
 (segment (start 147.32 99.06) (end 147.32 99.06) (width 0.25) (layer F.Cu) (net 31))
 (via (at 147.32 99.06) (size 0.8) (drill 0.4) (layers F.Cu B.Cu) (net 31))
 (segment (start 170.815 66.675) (end 168.275 69.215) (width 0.25) (layer B.Cu) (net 31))
 (segment (start 168.275 69.215) (end 168.275 71.12) (width 0.25) (layer B.Cu) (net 31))
 (segment (start 147.32 92.075) (end 147.32 99.06) (width 0.25) (layer B.Cu) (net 31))
 (segment (start 168.275 71.12) (end 147.32 92.075) (width 0.25) (layer B.Cu) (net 31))
 (segment (start 170.815 66.675) (end 173.99 63.5) (width 0.25) (layer B.Cu) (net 31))
 (segment (start 173.99 63.5) (end 208.915 63.5) (width 0.25) (layer B.Cu) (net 31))
 (segment (start 208.915 63.5) (end 214.63 69.215) (width 0.25) (layer B.Cu) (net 31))
 (segment (start 214.63 69.215) (end 214.63 69.215) (width 0.25) (layer B.Cu) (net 31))
 (via (at 214.63 69.215) (size 0.8) (drill 0.4) (layers F.Cu B.Cu) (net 31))
 (segment (start 214.63 69.215) (end 215.9 69.215) (width 0.25) (layer F.Cu) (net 31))
 (segment (start 222.885 76.2) (end 222.885 80.645) (width 0.25) (layer F.Cu) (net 31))
 (segment (start 215.9 69.215) (end 222.885 76.2) (width 0.25) (layer F.Cu) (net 31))
 (segment (start 214.63 88.265) (end 210.185 88.265) (width 0.25) (layer B.Cu) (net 31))
 (segment (start 218.44 84.455) (end 214.63 88.265) (width 0.25) (layer B.Cu) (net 31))
 (segment (start 222.25 84.455) (end 218.44 84.455) (width 0.25) (layer B.Cu) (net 31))
 (segment (start 222.885 83.82) (end 222.25 84.455) (width 0.25) (layer B.Cu) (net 31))
 (segment (start 222.885 80.645) (end 222.885 83.82) (width 0.25) (layer B.Cu) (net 31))
 (segment (start 164.189998 117.475) (end 165.735 117.475) (width 0.25) (layer F.Cu) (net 27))
 (segment (start 129.54 79.375) (end 159.385 109.22) (width 0.25) (layer F.Cu) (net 27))
 (segment (start 159.385 109.22) (end 159.385 112.670002) (width 0.25) (layer F.Cu) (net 27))
 (segment (start 122.555 79.375) (end 129.54 79.375) (width 0.25) (layer F.Cu) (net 27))
 (segment (start 159.385 112.670002) (end 164.189998 117.475) (width 0.25) (layer F.Cu) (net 27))
 (segment (start 120.65 81.28) (end 122.555 79.375) (width 0.25) (layer F.Cu) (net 27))
 (segment (start 120.65 83.185) (end 120.65 81.28) (width 0.25) (layer F.Cu) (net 27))
 (segment (start 220.345 86.36) (end 220.345 80.645) (width 0.25) (layer F.Cu) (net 25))
 (segment (start 195.58 111.125) (end 220.345 86.36) (width 0.25) (layer F.Cu) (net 25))
 (segment (start 182.245 111.125) (end 195.58 111.125) (width 0.25) (layer F.Cu) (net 25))
 (segment (start 180.975 112.395) (end 182.245 111.125) (width 0.25) (layer F.Cu) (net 25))
 (segment (start 165.735 112.395) (end 180.975 112.395) (width 0.25) (layer F.Cu) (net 25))
 (segment (start 187.325 108.585) (end 168.464998 108.585) (width 0.25) (layer F.Cu) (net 24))
 (segment (start 205.105 90.805) (end 187.325 108.585) (width 0.25) (layer F.Cu) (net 24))
 (segment (start 167.194998 109.855) (end 165.735 109.855) (width 0.25) (layer F.Cu) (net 24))
 (segment (start 168.464998 108.585) (end 167.194998 109.855) (width 0.25) (layer F.Cu) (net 24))
 (segment (start 210.185 90.805) (end 205.105 90.805) (width 0.25) (layer F.Cu) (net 24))
 (segment (start 135.89 129.54) (end 138.43 127) (width 0.25) (layer F.Cu) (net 11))
 (segment (start 121.92 128.27) (end 123.19 129.54) (width 0.25) (layer F.Cu) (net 11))
 (segment (start 123.19 129.54) (end 135.89 129.54) (width 0.25) (layer F.Cu) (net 11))
 (segment (start 138.43 127) (end 140.97 127) (width 0.25) (layer F.Cu) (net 11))
 (segment (start 121.92 123.19) (end 121.92 128.27) (width 0.25) (layer F.Cu) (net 11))
 (segment (start 123.8504 121.2596) (end 121.92 123.19) (width 0.25) (layer F.Cu) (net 11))
 (segment (start 126.5682 121.2596) (end 123.8504 121.2596) (width 0.25) (layer F.Cu) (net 11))
 (segment (start 226.165 65.935) (end 226.165 65.575) (width 0.25) (layer B.Cu) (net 11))
 (segment (start 222.25 69.85) (end 226.165 65.935) (width 0.25) (layer B.Cu) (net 11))
 (segment (start 220.345 69.85) (end 222.25 69.85) (width 0.25) (layer B.Cu) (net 11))
 (segment (start 205.105 85.09) (end 220.345 69.85) (width 0.25) (layer B.Cu) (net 11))
 (segment (start 205.105 116.84) (end 205.105 85.09) (width 0.25) (layer B.Cu) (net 11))
 (segment (start 185.42 136.525) (end 205.105 116.84) (width 0.25) (layer B.Cu) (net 11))
 (segment (start 140.97 127) (end 151.13 127) (width 0.25) (layer B.Cu) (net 11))
 (segment (start 160.655 136.525) (end 185.42 136.525) (width 0.25) (layer B.Cu) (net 11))
 (segment (start 151.13 127) (end 160.655 136.525) (width 0.25) (layer B.Cu) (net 11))
 (segment (start 165.735 84.455) (end 165.735 82.55) (width 0.25) (layer B.Cu) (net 2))
 (segment (start 165.735 82.55) (end 167.64 80.645) (width 0.25) (layer B.Cu) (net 2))
 (segment (start 178.635 80.645) (end 193.875 65.405) (width 0.25) (layer B.Cu) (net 2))
 (segment (start 167.64 80.645) (end 178.635 80.645) (width 0.25) (layer B.Cu) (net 2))
 (segment (start 183.515 84.455) (end 183.515 82.55) (width 0.25) (layer F.Cu) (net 3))
 (segment (start 183.515 82.55) (end 180.34 79.375) (width 0.25) (layer F.Cu) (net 3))
 (segment (start 180.34 79.375) (end 161.925 79.375) (width 0.25) (layer F.Cu) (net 3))
 (segment (start 161.925 79.375) (end 159.385 76.835) (width 0.25) (layer F.Cu) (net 3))
 (segment (start 159.385 69.295) (end 155.575 65.485) (width 0.25) (layer F.Cu) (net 3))
 (segment (start 159.385 76.835) (end 159.385 69.295) (width 0.25) (layer F.Cu) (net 3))
 (segment (start 156.845 82.55) (end 153.035 78.74) (width 0.25) (layer F.Cu) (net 6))
 (segment (start 166.37 82.55) (end 156.845 82.55) (width 0.25) (layer F.Cu) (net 6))
 (segment (start 183.515 99.695) (end 166.37 82.55) (width 0.25) (layer F.Cu) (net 6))
 (segment (start 196.215 95.885) (end 196.215 79.375) (width 0.25) (layer F.Cu) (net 4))
 (segment (start 187.325 104.775) (end 196.215 95.885) (width 0.25) (layer F.Cu) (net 4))
 (segment (start 183.515 104.775) (end 187.325 104.775) (width 0.25) (layer F.Cu) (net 4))
 (segment (start 145.415 78.74) (end 145.415 72.39) (width 0.25) (layer F.Cu) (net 7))
 (segment (start 151.13 66.675) (end 151.13 55.88) (width 0.25) (layer F.Cu) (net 7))
 (segment (start 145.415 72.39) (end 151.13 66.675) (width 0.25) (layer F.Cu) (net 7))
 (segment (start 203.835 57.785) (end 201.93 55.88) (width 0.25) (layer F.Cu) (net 5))
 (segment (start 203.835 79.375) (end 203.835 57.785) (width 0.25) (layer F.Cu) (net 5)))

